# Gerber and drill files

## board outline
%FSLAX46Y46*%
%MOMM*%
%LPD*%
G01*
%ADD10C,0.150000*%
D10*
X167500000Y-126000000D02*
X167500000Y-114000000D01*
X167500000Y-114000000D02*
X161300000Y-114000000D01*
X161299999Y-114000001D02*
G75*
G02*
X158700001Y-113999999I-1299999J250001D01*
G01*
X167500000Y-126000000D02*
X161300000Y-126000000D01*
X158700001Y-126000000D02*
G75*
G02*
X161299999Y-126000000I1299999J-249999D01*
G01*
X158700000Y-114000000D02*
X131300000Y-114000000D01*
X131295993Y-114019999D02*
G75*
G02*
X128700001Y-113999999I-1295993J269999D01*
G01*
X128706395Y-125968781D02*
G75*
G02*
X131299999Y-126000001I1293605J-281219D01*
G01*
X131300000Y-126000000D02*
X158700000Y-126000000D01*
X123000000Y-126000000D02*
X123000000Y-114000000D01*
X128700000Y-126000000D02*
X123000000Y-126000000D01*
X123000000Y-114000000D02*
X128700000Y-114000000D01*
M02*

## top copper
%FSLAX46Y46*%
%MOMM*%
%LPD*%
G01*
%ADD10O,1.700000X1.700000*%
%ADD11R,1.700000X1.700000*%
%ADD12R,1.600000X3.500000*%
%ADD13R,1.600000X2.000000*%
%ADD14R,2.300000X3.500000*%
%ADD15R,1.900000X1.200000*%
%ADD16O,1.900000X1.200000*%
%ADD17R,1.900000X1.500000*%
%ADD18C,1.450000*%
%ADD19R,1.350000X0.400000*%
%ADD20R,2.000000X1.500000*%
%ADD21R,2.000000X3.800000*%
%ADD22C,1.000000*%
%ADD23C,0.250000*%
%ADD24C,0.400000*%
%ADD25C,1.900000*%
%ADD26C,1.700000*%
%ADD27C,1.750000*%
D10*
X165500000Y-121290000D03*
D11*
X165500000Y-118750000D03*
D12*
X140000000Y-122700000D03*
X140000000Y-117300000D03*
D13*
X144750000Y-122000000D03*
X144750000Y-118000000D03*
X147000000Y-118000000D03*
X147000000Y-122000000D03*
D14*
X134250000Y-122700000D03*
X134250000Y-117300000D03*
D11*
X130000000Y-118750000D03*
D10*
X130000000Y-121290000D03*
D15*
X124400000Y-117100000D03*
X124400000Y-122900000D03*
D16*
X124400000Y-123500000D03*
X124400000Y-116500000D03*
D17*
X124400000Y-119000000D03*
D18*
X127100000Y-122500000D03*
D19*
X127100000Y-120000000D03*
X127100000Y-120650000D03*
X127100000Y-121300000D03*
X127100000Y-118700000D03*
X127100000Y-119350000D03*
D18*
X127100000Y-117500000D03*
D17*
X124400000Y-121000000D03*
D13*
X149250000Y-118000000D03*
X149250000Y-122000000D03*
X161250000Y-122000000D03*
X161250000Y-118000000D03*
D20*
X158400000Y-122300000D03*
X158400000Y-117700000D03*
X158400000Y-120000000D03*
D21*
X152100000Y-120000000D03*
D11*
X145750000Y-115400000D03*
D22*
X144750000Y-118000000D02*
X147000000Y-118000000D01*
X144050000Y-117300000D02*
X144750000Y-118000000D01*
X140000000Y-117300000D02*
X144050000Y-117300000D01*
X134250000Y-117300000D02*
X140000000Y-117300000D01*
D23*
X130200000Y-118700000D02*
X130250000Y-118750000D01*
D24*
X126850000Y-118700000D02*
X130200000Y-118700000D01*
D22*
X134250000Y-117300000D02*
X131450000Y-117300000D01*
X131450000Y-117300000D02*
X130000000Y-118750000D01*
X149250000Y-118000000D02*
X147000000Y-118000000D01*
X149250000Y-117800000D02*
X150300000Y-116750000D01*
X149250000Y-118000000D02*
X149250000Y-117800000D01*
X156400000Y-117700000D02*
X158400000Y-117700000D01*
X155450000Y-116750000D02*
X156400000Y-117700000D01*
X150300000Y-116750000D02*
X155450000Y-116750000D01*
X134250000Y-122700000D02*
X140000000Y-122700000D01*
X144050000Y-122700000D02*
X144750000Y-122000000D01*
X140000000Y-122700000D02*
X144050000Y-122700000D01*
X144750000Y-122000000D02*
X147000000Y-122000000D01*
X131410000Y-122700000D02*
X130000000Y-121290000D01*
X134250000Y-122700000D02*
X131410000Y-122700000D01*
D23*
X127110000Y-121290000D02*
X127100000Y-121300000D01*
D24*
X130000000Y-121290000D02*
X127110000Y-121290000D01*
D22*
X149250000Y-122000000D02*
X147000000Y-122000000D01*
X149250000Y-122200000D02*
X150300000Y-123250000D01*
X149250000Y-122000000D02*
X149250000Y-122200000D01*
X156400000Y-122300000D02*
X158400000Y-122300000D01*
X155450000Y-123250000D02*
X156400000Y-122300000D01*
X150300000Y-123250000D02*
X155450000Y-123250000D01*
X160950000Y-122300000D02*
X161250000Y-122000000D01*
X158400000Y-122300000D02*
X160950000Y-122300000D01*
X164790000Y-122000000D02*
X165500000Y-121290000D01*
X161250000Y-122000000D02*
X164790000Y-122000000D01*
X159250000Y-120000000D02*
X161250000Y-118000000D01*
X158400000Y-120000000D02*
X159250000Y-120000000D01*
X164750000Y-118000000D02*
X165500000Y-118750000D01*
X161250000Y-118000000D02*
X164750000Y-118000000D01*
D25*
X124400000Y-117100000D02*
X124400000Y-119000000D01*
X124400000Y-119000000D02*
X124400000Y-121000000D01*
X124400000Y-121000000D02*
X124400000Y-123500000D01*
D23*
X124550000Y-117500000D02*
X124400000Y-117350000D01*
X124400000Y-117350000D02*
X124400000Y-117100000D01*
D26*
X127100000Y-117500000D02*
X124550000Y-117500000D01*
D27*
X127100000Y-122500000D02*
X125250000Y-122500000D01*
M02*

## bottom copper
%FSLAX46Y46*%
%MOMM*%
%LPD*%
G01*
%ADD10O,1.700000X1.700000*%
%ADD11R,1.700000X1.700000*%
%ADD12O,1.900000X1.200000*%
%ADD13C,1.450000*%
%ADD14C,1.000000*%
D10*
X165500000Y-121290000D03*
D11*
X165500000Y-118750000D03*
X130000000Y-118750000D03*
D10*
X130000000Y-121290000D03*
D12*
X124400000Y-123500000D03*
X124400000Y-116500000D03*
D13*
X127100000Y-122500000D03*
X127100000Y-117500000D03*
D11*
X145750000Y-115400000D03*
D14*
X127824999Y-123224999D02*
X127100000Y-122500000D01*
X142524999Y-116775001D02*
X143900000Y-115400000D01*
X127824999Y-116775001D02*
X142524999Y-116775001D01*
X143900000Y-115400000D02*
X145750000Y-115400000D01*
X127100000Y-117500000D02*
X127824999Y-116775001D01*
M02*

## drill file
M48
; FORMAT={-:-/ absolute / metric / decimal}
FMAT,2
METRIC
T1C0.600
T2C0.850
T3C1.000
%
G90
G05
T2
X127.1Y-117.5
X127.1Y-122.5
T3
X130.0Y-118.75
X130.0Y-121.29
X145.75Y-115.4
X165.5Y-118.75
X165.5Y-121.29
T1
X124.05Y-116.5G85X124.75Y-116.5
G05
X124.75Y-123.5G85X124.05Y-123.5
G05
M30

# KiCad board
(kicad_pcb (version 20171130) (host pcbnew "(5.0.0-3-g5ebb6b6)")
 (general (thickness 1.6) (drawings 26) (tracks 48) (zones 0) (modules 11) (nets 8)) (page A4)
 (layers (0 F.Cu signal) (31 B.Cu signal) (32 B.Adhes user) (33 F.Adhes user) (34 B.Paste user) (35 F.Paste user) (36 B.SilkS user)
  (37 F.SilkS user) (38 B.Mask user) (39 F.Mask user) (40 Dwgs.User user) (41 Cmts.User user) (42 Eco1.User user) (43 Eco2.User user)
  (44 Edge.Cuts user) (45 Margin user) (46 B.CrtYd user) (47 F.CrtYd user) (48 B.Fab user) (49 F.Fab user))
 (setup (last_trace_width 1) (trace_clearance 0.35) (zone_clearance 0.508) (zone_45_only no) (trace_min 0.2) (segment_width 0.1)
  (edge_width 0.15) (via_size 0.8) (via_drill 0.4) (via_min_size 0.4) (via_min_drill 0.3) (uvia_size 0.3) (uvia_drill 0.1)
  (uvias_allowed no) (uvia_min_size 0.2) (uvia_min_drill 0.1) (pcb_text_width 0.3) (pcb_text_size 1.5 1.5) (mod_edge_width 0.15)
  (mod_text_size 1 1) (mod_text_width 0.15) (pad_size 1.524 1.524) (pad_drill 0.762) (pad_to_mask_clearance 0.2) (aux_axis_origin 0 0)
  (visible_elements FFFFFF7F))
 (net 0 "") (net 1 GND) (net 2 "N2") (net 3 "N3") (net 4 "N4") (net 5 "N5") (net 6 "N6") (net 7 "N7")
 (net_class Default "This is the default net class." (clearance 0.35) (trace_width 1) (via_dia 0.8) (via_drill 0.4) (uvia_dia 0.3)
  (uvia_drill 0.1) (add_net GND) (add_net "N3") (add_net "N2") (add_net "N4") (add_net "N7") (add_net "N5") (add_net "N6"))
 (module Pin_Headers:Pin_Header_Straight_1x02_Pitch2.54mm (layer F.Cu) (at 165.5 118.75)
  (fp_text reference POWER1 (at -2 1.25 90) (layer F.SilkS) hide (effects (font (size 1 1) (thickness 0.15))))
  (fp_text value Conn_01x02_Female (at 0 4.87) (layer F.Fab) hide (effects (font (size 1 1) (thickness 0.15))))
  (pad 2 thru_hole oval (at 0 2.54) (size 1.7 1.7) (drill 1) (layers *.Cu *.Mask) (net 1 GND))
  (pad 1 thru_hole rect (at 0 0) (size 1.7 1.7) (drill 1) (layers *.Cu *.Mask) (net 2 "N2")))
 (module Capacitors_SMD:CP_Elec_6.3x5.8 (layer F.Cu) (at 140 120 270)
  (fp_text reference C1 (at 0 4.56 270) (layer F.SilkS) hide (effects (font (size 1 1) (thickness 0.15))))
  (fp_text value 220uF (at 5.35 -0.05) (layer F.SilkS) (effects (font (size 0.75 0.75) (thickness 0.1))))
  (pad 2 smd rect (at 2.7 0 90) (size 3.5 1.6) (layers F.Cu F.Paste F.Mask) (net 1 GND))
  (pad 1 smd rect (at -2.7 0 90) (size 3.5 1.6) (layers F.Cu F.Paste F.Mask) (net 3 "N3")))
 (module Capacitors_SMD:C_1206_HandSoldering (layer F.Cu) (at 144.75 120 270)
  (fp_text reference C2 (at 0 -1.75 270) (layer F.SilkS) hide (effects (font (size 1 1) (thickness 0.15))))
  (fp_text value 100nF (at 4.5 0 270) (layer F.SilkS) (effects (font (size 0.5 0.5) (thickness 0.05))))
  (pad 2 smd rect (at 2 0 270) (size 2 1.6) (layers F.Cu F.Paste F.Mask) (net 1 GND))
  (pad 1 smd rect (at -2 0 270) (size 2 1.6) (layers F.Cu F.Paste F.Mask) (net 3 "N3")))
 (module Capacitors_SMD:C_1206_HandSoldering (layer F.Cu) (at 147 120 270)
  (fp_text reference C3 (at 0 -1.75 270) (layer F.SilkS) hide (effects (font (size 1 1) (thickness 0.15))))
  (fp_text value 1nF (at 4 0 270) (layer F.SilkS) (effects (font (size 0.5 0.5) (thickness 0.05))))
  (pad 1 smd rect (at -2 0 270) (size 2 1.6) (layers F.Cu F.Paste F.Mask) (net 3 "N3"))
  (pad 2 smd rect (at 2 0 270) (size 2 1.6) (layers F.Cu F.Paste F.Mask) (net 1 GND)))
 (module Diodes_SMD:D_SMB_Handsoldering (layer F.Cu) (at 134.25 120 270)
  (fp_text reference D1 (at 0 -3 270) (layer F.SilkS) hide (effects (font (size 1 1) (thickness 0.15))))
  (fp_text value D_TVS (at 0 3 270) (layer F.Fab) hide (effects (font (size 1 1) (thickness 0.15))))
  (pad 2 smd rect (at 2.7 0 270) (size 3.5 2.3) (layers F.Cu F.Paste F.Mask) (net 1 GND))
  (pad 1 smd rect (at -2.7 0 270) (size 3.5 2.3) (layers F.Cu F.Paste F.Mask) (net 3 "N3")))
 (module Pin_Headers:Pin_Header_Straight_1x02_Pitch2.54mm (layer F.Cu) (at 130 118.75)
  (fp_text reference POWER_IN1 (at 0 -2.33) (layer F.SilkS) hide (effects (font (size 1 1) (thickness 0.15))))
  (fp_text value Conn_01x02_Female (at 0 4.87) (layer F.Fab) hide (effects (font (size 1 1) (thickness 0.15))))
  (pad 1 thru_hole rect (at 0 0) (size 1.7 1.7) (drill 1) (layers *.Cu *.Mask) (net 3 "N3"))
  (pad 2 thru_hole oval (at 0 2.54) (size 1.7 1.7) (drill 1) (layers *.Cu *.Mask) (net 1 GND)))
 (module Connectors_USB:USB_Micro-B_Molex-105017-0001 (layer F.Cu) (at 124.75 120 270)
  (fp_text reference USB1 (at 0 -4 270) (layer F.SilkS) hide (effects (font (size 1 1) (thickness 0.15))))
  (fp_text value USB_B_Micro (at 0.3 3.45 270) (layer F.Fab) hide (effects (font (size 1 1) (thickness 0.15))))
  (pad 6 smd rect (at -2.9 0.35 270) (size 1.2 1.9) (layers F.Cu F.Mask) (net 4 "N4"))
  (pad 6 smd rect (at 2.9 0.35 270) (size 1.2 1.9) (layers F.Cu F.Mask) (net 4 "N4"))
  (pad 6 thru_hole oval (at 3.5 0.35 270) (size 1.2 1.9) (drill oval 0.6 1.3) (layers *.Cu *.Mask) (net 4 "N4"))
  (pad 6 thru_hole oval (at -3.5 0.35 90) (size 1.2 1.9) (drill oval 0.6 1.3) (layers *.Cu *.Mask) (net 4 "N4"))
  (pad 6 smd rect (at -1 0.35 270) (size 1.5 1.9) (layers F.Cu F.Paste F.Mask) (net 4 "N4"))
  (pad 6 thru_hole circle (at 2.5 -2.35 270) (size 1.45 1.45) (drill 0.85) (layers *.Cu *.Mask) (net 4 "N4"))
  (pad 3 smd rect (at 0 -2.35 270) (size 0.4 1.35) (layers F.Cu F.Paste F.Mask) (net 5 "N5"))
  (pad 4 smd rect (at 0.65 -2.35 270) (size 0.4 1.35) (layers F.Cu F.Paste F.Mask) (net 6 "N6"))
  (pad 5 smd rect (at 1.3 -2.35 270) (size 0.4 1.35) (layers F.Cu F.Paste F.Mask) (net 1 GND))
  (pad 1 smd rect (at -1.3 -2.35 270) (size 0.4 1.35) (layers F.Cu F.Paste F.Mask) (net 3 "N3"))
  (pad 2 smd rect (at -0.65 -2.35 270) (size 0.4 1.35) (layers F.Cu F.Paste F.Mask) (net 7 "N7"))
  (pad 6 thru_hole circle (at -2.5 -2.35 270) (size 1.45 1.45) (drill 0.85) (layers *.Cu *.Mask) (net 4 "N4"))
  (pad 6 smd rect (at 1 0.35 270) (size 1.5 1.9) (layers F.Cu F.Paste F.Mask) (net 4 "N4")))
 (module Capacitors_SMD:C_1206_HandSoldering (layer F.Cu) (at 149.25 120 270)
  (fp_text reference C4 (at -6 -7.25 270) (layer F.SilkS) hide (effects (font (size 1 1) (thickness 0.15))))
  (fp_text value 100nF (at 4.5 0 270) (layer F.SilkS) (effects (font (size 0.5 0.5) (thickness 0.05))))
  (pad 1 smd rect (at -2 0 270) (size 2 1.6) (layers F.Cu F.Paste F.Mask) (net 3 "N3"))
  (pad 2 smd rect (at 2 0 270) (size 2 1.6) (layers F.Cu F.Paste F.Mask) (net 1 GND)))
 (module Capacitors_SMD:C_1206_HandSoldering (layer F.Cu) (at 161.25 120 270)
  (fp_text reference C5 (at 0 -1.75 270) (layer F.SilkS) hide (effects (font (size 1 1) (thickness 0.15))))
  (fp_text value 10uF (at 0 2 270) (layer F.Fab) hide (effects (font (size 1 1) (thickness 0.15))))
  (pad 2 smd rect (at 2 0 270) (size 2 1.6) (layers F.Cu F.Paste F.Mask) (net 1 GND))
  (pad 1 smd rect (at -2 0 270) (size 2 1.6) (layers F.Cu F.Paste F.Mask) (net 2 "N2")))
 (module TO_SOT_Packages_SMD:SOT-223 (layer F.Cu) (at 155.25 120 180)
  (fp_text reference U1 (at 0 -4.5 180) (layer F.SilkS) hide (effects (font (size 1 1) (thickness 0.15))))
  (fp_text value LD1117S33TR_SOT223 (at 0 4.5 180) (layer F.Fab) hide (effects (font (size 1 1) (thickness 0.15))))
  (pad 1 smd rect (at -3.15 -2.3 180) (size 2 1.5) (layers F.Cu F.Paste F.Mask) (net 1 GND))
  (pad 3 smd rect (at -3.15 2.3 180) (size 2 1.5) (layers F.Cu F.Paste F.Mask) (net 3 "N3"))
  (pad 2 smd rect (at -3.15 0 180) (size 2 1.5) (layers F.Cu F.Paste F.Mask) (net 2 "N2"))
  (pad 4 smd rect (at 3.15 0 180) (size 2 3.8) (layers F.Cu F.Paste F.Mask)))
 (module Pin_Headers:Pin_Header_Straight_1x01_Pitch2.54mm (layer F.Cu) (at 145.75 115.4)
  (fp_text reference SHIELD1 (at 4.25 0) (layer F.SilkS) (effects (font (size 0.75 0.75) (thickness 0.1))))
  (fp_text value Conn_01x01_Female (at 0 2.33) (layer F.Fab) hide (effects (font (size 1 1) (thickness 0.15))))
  (pad 1 thru_hole rect (at 0 0) (size 1.7 1.7) (drill 1) (layers *.Cu *.Mask) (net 4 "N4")))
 (gr_line (start 167.5 126) (end 167.5 114) (layer Edge.Cuts) (width 0.15))
 (gr_line (start 167.5 114) (end 161.3 114) (layer Edge.Cuts) (width 0.15))
 (gr_arc (start 160 113.75) (end 158.700001 113.999999) (angle -158.2289459) (layer Edge.Cuts) (width 0.15))
 (gr_line (start 167.5 126) (end 161.3 126) (layer Edge.Cuts) (width 0.15))
 (gr_arc (start 160 126.249999) (end 161.299999 126) (angle -158.2290064) (layer Edge.Cuts) (width 0.15))
 (gr_line (start 158.7 114) (end 131.3 114) (layer Edge.Cuts) (width 0.15))
 (gr_arc (start 130 113.75) (end 128.700001 113.999999) (angle -157.346184) (layer Edge.Cuts) (width 0.15))
 (gr_arc (start 130 126.25) (end 131.299999 126.000001) (angle -156.8496992) (layer Edge.Cuts) (width 0.15))
 (gr_line (start 131.3 126) (end 158.7 126) (layer Edge.Cuts) (width 0.15))
 (gr_line (start 123 126) (end 123 114) (layer Edge.Cuts) (width 0.15))
 (gr_line (start 128.7 126) (end 123 126) (layer Edge.Cuts) (width 0.15))
 (gr_line (start 123 114) (end 128.7 114) (layer Edge.Cuts) (width 0.15))
 (segment (start 144.75 118) (end 147 118) (width 1) (layer F.Cu) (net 3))
 (segment (start 144.05 117.3) (end 144.75 118) (width 1) (layer F.Cu) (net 3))
 (segment (start 140 117.3) (end 144.05 117.3) (width 1) (layer F.Cu) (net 3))
 (segment (start 134.25 117.3) (end 140 117.3) (width 1) (layer F.Cu) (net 3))
 (segment (start 130.2 118.7) (end 130.25 118.75) (width 0.25) (layer F.Cu) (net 3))
 (segment (start 126.85 118.7) (end 130.2 118.7) (width 0.4) (layer F.Cu) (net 3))
 (segment (start 134.25 117.3) (end 131.45 117.3) (width 1) (layer F.Cu) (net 3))
 (segment (start 131.45 117.3) (end 130 118.75) (width 1) (layer F.Cu) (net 3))
 (segment (start 149.25 118) (end 147 118) (width 1) (layer F.Cu) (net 3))
 (segment (start 149.25 117.8) (end 150.3 116.75) (width 1) (layer F.Cu) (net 3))
 (segment (start 149.25 118) (end 149.25 117.8) (width 1) (layer F.Cu) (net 3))
 (segment (start 156.4 117.7) (end 158.4 117.7) (width 1) (layer F.Cu) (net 3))
 (segment (start 155.45 116.75) (end 156.4 117.7) (width 1) (layer F.Cu) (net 3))
 (segment (start 150.3 116.75) (end 155.45 116.75) (width 1) (layer F.Cu) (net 3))
 (segment (start 134.25 122.7) (end 140 122.7) (width 1) (layer F.Cu) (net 1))
 (segment (start 144.05 122.7) (end 144.75 122) (width 1) (layer F.Cu) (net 1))
 (segment (start 140 122.7) (end 144.05 122.7) (width 1) (layer F.Cu) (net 1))
 (segment (start 144.75 122) (end 147 122) (width 1) (layer F.Cu) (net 1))
 (segment (start 131.41 122.7) (end 130 121.29) (width 1) (layer F.Cu) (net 1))
 (segment (start 134.25 122.7) (end 131.41 122.7) (width 1) (layer F.Cu) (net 1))
 (segment (start 127.11 121.29) (end 127.1 121.3) (width 0.25) (layer F.Cu) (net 1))
 (segment (start 130 121.29) (end 127.11 121.29) (width 0.4) (layer F.Cu) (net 1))
 (segment (start 149.25 122) (end 147 122) (width 1) (layer F.Cu) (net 1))
 (segment (start 149.25 122.2) (end 150.3 123.25) (width 1) (layer F.Cu) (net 1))
 (segment (start 149.25 122) (end 149.25 122.2) (width 1) (layer F.Cu) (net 1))
 (segment (start 156.4 122.3) (end 158.4 122.3) (width 1) (layer F.Cu) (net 1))
 (segment (start 155.45 123.25) (end 156.4 122.3) (width 1) (layer F.Cu) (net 1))
 (segment (start 150.3 123.25) (end 155.45 123.25) (width 1) (layer F.Cu) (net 1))
 (segment (start 160.95 122.3) (end 161.25 122) (width 1) (layer F.Cu) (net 1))
 (segment (start 158.4 122.3) (end 160.95 122.3) (width 1) (layer F.Cu) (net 1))
 (segment (start 164.79 122) (end 165.5 121.29) (width 1) (layer F.Cu) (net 1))
 (segment (start 161.25 122) (end 164.79 122) (width 1) (layer F.Cu) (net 1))
 (segment (start 159.25 120) (end 161.25 118) (width 1) (layer F.Cu) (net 2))
 (segment (start 158.4 120) (end 159.25 120) (width 1) (layer F.Cu) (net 2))
 (segment (start 164.75 118) (end 165.5 118.75) (width 1) (layer F.Cu) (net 2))
 (segment (start 161.25 118) (end 164.75 118) (width 1) (layer F.Cu) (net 2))
 (segment (start 124.4 117.1) (end 124.4 119) (width 1.9) (layer F.Cu) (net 4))
 (segment (start 124.4 119) (end 124.4 121) (width 1.9) (layer F.Cu) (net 4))
 (segment (start 124.4 121) (end 124.4 123.5) (width 1.9) (layer F.Cu) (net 4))
 (segment (start 124.55 117.5) (end 124.4 117.35) (width 0.25) (layer F.Cu) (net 4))
 (segment (start 124.4 117.35) (end 124.4 117.1) (width 0.25) (layer F.Cu) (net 4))
 (segment (start 127.1 117.5) (end 124.55 117.5) (width 1.7) (layer F.Cu) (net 4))
 (segment (start 127.1 122.5) (end 125.25 122.5) (width 1.75) (layer F.Cu) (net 4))
 (segment (start 127.824999 123.224999) (end 127.1 122.5) (width 1) (layer B.Cu) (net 4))
 (segment (start 142.524999 116.775001) (end 143.9 115.4) (width 1) (layer B.Cu) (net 4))
 (segment (start 127.824999 116.775001) (end 142.524999 116.775001) (width 1) (layer B.Cu) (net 4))
 (segment (start 143.9 115.4) (end 145.75 115.4) (width 1) (layer B.Cu) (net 4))
 (segment (start 127.1 117.5) (end 127.824999 116.775001) (width 1) (layer B.Cu) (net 4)))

